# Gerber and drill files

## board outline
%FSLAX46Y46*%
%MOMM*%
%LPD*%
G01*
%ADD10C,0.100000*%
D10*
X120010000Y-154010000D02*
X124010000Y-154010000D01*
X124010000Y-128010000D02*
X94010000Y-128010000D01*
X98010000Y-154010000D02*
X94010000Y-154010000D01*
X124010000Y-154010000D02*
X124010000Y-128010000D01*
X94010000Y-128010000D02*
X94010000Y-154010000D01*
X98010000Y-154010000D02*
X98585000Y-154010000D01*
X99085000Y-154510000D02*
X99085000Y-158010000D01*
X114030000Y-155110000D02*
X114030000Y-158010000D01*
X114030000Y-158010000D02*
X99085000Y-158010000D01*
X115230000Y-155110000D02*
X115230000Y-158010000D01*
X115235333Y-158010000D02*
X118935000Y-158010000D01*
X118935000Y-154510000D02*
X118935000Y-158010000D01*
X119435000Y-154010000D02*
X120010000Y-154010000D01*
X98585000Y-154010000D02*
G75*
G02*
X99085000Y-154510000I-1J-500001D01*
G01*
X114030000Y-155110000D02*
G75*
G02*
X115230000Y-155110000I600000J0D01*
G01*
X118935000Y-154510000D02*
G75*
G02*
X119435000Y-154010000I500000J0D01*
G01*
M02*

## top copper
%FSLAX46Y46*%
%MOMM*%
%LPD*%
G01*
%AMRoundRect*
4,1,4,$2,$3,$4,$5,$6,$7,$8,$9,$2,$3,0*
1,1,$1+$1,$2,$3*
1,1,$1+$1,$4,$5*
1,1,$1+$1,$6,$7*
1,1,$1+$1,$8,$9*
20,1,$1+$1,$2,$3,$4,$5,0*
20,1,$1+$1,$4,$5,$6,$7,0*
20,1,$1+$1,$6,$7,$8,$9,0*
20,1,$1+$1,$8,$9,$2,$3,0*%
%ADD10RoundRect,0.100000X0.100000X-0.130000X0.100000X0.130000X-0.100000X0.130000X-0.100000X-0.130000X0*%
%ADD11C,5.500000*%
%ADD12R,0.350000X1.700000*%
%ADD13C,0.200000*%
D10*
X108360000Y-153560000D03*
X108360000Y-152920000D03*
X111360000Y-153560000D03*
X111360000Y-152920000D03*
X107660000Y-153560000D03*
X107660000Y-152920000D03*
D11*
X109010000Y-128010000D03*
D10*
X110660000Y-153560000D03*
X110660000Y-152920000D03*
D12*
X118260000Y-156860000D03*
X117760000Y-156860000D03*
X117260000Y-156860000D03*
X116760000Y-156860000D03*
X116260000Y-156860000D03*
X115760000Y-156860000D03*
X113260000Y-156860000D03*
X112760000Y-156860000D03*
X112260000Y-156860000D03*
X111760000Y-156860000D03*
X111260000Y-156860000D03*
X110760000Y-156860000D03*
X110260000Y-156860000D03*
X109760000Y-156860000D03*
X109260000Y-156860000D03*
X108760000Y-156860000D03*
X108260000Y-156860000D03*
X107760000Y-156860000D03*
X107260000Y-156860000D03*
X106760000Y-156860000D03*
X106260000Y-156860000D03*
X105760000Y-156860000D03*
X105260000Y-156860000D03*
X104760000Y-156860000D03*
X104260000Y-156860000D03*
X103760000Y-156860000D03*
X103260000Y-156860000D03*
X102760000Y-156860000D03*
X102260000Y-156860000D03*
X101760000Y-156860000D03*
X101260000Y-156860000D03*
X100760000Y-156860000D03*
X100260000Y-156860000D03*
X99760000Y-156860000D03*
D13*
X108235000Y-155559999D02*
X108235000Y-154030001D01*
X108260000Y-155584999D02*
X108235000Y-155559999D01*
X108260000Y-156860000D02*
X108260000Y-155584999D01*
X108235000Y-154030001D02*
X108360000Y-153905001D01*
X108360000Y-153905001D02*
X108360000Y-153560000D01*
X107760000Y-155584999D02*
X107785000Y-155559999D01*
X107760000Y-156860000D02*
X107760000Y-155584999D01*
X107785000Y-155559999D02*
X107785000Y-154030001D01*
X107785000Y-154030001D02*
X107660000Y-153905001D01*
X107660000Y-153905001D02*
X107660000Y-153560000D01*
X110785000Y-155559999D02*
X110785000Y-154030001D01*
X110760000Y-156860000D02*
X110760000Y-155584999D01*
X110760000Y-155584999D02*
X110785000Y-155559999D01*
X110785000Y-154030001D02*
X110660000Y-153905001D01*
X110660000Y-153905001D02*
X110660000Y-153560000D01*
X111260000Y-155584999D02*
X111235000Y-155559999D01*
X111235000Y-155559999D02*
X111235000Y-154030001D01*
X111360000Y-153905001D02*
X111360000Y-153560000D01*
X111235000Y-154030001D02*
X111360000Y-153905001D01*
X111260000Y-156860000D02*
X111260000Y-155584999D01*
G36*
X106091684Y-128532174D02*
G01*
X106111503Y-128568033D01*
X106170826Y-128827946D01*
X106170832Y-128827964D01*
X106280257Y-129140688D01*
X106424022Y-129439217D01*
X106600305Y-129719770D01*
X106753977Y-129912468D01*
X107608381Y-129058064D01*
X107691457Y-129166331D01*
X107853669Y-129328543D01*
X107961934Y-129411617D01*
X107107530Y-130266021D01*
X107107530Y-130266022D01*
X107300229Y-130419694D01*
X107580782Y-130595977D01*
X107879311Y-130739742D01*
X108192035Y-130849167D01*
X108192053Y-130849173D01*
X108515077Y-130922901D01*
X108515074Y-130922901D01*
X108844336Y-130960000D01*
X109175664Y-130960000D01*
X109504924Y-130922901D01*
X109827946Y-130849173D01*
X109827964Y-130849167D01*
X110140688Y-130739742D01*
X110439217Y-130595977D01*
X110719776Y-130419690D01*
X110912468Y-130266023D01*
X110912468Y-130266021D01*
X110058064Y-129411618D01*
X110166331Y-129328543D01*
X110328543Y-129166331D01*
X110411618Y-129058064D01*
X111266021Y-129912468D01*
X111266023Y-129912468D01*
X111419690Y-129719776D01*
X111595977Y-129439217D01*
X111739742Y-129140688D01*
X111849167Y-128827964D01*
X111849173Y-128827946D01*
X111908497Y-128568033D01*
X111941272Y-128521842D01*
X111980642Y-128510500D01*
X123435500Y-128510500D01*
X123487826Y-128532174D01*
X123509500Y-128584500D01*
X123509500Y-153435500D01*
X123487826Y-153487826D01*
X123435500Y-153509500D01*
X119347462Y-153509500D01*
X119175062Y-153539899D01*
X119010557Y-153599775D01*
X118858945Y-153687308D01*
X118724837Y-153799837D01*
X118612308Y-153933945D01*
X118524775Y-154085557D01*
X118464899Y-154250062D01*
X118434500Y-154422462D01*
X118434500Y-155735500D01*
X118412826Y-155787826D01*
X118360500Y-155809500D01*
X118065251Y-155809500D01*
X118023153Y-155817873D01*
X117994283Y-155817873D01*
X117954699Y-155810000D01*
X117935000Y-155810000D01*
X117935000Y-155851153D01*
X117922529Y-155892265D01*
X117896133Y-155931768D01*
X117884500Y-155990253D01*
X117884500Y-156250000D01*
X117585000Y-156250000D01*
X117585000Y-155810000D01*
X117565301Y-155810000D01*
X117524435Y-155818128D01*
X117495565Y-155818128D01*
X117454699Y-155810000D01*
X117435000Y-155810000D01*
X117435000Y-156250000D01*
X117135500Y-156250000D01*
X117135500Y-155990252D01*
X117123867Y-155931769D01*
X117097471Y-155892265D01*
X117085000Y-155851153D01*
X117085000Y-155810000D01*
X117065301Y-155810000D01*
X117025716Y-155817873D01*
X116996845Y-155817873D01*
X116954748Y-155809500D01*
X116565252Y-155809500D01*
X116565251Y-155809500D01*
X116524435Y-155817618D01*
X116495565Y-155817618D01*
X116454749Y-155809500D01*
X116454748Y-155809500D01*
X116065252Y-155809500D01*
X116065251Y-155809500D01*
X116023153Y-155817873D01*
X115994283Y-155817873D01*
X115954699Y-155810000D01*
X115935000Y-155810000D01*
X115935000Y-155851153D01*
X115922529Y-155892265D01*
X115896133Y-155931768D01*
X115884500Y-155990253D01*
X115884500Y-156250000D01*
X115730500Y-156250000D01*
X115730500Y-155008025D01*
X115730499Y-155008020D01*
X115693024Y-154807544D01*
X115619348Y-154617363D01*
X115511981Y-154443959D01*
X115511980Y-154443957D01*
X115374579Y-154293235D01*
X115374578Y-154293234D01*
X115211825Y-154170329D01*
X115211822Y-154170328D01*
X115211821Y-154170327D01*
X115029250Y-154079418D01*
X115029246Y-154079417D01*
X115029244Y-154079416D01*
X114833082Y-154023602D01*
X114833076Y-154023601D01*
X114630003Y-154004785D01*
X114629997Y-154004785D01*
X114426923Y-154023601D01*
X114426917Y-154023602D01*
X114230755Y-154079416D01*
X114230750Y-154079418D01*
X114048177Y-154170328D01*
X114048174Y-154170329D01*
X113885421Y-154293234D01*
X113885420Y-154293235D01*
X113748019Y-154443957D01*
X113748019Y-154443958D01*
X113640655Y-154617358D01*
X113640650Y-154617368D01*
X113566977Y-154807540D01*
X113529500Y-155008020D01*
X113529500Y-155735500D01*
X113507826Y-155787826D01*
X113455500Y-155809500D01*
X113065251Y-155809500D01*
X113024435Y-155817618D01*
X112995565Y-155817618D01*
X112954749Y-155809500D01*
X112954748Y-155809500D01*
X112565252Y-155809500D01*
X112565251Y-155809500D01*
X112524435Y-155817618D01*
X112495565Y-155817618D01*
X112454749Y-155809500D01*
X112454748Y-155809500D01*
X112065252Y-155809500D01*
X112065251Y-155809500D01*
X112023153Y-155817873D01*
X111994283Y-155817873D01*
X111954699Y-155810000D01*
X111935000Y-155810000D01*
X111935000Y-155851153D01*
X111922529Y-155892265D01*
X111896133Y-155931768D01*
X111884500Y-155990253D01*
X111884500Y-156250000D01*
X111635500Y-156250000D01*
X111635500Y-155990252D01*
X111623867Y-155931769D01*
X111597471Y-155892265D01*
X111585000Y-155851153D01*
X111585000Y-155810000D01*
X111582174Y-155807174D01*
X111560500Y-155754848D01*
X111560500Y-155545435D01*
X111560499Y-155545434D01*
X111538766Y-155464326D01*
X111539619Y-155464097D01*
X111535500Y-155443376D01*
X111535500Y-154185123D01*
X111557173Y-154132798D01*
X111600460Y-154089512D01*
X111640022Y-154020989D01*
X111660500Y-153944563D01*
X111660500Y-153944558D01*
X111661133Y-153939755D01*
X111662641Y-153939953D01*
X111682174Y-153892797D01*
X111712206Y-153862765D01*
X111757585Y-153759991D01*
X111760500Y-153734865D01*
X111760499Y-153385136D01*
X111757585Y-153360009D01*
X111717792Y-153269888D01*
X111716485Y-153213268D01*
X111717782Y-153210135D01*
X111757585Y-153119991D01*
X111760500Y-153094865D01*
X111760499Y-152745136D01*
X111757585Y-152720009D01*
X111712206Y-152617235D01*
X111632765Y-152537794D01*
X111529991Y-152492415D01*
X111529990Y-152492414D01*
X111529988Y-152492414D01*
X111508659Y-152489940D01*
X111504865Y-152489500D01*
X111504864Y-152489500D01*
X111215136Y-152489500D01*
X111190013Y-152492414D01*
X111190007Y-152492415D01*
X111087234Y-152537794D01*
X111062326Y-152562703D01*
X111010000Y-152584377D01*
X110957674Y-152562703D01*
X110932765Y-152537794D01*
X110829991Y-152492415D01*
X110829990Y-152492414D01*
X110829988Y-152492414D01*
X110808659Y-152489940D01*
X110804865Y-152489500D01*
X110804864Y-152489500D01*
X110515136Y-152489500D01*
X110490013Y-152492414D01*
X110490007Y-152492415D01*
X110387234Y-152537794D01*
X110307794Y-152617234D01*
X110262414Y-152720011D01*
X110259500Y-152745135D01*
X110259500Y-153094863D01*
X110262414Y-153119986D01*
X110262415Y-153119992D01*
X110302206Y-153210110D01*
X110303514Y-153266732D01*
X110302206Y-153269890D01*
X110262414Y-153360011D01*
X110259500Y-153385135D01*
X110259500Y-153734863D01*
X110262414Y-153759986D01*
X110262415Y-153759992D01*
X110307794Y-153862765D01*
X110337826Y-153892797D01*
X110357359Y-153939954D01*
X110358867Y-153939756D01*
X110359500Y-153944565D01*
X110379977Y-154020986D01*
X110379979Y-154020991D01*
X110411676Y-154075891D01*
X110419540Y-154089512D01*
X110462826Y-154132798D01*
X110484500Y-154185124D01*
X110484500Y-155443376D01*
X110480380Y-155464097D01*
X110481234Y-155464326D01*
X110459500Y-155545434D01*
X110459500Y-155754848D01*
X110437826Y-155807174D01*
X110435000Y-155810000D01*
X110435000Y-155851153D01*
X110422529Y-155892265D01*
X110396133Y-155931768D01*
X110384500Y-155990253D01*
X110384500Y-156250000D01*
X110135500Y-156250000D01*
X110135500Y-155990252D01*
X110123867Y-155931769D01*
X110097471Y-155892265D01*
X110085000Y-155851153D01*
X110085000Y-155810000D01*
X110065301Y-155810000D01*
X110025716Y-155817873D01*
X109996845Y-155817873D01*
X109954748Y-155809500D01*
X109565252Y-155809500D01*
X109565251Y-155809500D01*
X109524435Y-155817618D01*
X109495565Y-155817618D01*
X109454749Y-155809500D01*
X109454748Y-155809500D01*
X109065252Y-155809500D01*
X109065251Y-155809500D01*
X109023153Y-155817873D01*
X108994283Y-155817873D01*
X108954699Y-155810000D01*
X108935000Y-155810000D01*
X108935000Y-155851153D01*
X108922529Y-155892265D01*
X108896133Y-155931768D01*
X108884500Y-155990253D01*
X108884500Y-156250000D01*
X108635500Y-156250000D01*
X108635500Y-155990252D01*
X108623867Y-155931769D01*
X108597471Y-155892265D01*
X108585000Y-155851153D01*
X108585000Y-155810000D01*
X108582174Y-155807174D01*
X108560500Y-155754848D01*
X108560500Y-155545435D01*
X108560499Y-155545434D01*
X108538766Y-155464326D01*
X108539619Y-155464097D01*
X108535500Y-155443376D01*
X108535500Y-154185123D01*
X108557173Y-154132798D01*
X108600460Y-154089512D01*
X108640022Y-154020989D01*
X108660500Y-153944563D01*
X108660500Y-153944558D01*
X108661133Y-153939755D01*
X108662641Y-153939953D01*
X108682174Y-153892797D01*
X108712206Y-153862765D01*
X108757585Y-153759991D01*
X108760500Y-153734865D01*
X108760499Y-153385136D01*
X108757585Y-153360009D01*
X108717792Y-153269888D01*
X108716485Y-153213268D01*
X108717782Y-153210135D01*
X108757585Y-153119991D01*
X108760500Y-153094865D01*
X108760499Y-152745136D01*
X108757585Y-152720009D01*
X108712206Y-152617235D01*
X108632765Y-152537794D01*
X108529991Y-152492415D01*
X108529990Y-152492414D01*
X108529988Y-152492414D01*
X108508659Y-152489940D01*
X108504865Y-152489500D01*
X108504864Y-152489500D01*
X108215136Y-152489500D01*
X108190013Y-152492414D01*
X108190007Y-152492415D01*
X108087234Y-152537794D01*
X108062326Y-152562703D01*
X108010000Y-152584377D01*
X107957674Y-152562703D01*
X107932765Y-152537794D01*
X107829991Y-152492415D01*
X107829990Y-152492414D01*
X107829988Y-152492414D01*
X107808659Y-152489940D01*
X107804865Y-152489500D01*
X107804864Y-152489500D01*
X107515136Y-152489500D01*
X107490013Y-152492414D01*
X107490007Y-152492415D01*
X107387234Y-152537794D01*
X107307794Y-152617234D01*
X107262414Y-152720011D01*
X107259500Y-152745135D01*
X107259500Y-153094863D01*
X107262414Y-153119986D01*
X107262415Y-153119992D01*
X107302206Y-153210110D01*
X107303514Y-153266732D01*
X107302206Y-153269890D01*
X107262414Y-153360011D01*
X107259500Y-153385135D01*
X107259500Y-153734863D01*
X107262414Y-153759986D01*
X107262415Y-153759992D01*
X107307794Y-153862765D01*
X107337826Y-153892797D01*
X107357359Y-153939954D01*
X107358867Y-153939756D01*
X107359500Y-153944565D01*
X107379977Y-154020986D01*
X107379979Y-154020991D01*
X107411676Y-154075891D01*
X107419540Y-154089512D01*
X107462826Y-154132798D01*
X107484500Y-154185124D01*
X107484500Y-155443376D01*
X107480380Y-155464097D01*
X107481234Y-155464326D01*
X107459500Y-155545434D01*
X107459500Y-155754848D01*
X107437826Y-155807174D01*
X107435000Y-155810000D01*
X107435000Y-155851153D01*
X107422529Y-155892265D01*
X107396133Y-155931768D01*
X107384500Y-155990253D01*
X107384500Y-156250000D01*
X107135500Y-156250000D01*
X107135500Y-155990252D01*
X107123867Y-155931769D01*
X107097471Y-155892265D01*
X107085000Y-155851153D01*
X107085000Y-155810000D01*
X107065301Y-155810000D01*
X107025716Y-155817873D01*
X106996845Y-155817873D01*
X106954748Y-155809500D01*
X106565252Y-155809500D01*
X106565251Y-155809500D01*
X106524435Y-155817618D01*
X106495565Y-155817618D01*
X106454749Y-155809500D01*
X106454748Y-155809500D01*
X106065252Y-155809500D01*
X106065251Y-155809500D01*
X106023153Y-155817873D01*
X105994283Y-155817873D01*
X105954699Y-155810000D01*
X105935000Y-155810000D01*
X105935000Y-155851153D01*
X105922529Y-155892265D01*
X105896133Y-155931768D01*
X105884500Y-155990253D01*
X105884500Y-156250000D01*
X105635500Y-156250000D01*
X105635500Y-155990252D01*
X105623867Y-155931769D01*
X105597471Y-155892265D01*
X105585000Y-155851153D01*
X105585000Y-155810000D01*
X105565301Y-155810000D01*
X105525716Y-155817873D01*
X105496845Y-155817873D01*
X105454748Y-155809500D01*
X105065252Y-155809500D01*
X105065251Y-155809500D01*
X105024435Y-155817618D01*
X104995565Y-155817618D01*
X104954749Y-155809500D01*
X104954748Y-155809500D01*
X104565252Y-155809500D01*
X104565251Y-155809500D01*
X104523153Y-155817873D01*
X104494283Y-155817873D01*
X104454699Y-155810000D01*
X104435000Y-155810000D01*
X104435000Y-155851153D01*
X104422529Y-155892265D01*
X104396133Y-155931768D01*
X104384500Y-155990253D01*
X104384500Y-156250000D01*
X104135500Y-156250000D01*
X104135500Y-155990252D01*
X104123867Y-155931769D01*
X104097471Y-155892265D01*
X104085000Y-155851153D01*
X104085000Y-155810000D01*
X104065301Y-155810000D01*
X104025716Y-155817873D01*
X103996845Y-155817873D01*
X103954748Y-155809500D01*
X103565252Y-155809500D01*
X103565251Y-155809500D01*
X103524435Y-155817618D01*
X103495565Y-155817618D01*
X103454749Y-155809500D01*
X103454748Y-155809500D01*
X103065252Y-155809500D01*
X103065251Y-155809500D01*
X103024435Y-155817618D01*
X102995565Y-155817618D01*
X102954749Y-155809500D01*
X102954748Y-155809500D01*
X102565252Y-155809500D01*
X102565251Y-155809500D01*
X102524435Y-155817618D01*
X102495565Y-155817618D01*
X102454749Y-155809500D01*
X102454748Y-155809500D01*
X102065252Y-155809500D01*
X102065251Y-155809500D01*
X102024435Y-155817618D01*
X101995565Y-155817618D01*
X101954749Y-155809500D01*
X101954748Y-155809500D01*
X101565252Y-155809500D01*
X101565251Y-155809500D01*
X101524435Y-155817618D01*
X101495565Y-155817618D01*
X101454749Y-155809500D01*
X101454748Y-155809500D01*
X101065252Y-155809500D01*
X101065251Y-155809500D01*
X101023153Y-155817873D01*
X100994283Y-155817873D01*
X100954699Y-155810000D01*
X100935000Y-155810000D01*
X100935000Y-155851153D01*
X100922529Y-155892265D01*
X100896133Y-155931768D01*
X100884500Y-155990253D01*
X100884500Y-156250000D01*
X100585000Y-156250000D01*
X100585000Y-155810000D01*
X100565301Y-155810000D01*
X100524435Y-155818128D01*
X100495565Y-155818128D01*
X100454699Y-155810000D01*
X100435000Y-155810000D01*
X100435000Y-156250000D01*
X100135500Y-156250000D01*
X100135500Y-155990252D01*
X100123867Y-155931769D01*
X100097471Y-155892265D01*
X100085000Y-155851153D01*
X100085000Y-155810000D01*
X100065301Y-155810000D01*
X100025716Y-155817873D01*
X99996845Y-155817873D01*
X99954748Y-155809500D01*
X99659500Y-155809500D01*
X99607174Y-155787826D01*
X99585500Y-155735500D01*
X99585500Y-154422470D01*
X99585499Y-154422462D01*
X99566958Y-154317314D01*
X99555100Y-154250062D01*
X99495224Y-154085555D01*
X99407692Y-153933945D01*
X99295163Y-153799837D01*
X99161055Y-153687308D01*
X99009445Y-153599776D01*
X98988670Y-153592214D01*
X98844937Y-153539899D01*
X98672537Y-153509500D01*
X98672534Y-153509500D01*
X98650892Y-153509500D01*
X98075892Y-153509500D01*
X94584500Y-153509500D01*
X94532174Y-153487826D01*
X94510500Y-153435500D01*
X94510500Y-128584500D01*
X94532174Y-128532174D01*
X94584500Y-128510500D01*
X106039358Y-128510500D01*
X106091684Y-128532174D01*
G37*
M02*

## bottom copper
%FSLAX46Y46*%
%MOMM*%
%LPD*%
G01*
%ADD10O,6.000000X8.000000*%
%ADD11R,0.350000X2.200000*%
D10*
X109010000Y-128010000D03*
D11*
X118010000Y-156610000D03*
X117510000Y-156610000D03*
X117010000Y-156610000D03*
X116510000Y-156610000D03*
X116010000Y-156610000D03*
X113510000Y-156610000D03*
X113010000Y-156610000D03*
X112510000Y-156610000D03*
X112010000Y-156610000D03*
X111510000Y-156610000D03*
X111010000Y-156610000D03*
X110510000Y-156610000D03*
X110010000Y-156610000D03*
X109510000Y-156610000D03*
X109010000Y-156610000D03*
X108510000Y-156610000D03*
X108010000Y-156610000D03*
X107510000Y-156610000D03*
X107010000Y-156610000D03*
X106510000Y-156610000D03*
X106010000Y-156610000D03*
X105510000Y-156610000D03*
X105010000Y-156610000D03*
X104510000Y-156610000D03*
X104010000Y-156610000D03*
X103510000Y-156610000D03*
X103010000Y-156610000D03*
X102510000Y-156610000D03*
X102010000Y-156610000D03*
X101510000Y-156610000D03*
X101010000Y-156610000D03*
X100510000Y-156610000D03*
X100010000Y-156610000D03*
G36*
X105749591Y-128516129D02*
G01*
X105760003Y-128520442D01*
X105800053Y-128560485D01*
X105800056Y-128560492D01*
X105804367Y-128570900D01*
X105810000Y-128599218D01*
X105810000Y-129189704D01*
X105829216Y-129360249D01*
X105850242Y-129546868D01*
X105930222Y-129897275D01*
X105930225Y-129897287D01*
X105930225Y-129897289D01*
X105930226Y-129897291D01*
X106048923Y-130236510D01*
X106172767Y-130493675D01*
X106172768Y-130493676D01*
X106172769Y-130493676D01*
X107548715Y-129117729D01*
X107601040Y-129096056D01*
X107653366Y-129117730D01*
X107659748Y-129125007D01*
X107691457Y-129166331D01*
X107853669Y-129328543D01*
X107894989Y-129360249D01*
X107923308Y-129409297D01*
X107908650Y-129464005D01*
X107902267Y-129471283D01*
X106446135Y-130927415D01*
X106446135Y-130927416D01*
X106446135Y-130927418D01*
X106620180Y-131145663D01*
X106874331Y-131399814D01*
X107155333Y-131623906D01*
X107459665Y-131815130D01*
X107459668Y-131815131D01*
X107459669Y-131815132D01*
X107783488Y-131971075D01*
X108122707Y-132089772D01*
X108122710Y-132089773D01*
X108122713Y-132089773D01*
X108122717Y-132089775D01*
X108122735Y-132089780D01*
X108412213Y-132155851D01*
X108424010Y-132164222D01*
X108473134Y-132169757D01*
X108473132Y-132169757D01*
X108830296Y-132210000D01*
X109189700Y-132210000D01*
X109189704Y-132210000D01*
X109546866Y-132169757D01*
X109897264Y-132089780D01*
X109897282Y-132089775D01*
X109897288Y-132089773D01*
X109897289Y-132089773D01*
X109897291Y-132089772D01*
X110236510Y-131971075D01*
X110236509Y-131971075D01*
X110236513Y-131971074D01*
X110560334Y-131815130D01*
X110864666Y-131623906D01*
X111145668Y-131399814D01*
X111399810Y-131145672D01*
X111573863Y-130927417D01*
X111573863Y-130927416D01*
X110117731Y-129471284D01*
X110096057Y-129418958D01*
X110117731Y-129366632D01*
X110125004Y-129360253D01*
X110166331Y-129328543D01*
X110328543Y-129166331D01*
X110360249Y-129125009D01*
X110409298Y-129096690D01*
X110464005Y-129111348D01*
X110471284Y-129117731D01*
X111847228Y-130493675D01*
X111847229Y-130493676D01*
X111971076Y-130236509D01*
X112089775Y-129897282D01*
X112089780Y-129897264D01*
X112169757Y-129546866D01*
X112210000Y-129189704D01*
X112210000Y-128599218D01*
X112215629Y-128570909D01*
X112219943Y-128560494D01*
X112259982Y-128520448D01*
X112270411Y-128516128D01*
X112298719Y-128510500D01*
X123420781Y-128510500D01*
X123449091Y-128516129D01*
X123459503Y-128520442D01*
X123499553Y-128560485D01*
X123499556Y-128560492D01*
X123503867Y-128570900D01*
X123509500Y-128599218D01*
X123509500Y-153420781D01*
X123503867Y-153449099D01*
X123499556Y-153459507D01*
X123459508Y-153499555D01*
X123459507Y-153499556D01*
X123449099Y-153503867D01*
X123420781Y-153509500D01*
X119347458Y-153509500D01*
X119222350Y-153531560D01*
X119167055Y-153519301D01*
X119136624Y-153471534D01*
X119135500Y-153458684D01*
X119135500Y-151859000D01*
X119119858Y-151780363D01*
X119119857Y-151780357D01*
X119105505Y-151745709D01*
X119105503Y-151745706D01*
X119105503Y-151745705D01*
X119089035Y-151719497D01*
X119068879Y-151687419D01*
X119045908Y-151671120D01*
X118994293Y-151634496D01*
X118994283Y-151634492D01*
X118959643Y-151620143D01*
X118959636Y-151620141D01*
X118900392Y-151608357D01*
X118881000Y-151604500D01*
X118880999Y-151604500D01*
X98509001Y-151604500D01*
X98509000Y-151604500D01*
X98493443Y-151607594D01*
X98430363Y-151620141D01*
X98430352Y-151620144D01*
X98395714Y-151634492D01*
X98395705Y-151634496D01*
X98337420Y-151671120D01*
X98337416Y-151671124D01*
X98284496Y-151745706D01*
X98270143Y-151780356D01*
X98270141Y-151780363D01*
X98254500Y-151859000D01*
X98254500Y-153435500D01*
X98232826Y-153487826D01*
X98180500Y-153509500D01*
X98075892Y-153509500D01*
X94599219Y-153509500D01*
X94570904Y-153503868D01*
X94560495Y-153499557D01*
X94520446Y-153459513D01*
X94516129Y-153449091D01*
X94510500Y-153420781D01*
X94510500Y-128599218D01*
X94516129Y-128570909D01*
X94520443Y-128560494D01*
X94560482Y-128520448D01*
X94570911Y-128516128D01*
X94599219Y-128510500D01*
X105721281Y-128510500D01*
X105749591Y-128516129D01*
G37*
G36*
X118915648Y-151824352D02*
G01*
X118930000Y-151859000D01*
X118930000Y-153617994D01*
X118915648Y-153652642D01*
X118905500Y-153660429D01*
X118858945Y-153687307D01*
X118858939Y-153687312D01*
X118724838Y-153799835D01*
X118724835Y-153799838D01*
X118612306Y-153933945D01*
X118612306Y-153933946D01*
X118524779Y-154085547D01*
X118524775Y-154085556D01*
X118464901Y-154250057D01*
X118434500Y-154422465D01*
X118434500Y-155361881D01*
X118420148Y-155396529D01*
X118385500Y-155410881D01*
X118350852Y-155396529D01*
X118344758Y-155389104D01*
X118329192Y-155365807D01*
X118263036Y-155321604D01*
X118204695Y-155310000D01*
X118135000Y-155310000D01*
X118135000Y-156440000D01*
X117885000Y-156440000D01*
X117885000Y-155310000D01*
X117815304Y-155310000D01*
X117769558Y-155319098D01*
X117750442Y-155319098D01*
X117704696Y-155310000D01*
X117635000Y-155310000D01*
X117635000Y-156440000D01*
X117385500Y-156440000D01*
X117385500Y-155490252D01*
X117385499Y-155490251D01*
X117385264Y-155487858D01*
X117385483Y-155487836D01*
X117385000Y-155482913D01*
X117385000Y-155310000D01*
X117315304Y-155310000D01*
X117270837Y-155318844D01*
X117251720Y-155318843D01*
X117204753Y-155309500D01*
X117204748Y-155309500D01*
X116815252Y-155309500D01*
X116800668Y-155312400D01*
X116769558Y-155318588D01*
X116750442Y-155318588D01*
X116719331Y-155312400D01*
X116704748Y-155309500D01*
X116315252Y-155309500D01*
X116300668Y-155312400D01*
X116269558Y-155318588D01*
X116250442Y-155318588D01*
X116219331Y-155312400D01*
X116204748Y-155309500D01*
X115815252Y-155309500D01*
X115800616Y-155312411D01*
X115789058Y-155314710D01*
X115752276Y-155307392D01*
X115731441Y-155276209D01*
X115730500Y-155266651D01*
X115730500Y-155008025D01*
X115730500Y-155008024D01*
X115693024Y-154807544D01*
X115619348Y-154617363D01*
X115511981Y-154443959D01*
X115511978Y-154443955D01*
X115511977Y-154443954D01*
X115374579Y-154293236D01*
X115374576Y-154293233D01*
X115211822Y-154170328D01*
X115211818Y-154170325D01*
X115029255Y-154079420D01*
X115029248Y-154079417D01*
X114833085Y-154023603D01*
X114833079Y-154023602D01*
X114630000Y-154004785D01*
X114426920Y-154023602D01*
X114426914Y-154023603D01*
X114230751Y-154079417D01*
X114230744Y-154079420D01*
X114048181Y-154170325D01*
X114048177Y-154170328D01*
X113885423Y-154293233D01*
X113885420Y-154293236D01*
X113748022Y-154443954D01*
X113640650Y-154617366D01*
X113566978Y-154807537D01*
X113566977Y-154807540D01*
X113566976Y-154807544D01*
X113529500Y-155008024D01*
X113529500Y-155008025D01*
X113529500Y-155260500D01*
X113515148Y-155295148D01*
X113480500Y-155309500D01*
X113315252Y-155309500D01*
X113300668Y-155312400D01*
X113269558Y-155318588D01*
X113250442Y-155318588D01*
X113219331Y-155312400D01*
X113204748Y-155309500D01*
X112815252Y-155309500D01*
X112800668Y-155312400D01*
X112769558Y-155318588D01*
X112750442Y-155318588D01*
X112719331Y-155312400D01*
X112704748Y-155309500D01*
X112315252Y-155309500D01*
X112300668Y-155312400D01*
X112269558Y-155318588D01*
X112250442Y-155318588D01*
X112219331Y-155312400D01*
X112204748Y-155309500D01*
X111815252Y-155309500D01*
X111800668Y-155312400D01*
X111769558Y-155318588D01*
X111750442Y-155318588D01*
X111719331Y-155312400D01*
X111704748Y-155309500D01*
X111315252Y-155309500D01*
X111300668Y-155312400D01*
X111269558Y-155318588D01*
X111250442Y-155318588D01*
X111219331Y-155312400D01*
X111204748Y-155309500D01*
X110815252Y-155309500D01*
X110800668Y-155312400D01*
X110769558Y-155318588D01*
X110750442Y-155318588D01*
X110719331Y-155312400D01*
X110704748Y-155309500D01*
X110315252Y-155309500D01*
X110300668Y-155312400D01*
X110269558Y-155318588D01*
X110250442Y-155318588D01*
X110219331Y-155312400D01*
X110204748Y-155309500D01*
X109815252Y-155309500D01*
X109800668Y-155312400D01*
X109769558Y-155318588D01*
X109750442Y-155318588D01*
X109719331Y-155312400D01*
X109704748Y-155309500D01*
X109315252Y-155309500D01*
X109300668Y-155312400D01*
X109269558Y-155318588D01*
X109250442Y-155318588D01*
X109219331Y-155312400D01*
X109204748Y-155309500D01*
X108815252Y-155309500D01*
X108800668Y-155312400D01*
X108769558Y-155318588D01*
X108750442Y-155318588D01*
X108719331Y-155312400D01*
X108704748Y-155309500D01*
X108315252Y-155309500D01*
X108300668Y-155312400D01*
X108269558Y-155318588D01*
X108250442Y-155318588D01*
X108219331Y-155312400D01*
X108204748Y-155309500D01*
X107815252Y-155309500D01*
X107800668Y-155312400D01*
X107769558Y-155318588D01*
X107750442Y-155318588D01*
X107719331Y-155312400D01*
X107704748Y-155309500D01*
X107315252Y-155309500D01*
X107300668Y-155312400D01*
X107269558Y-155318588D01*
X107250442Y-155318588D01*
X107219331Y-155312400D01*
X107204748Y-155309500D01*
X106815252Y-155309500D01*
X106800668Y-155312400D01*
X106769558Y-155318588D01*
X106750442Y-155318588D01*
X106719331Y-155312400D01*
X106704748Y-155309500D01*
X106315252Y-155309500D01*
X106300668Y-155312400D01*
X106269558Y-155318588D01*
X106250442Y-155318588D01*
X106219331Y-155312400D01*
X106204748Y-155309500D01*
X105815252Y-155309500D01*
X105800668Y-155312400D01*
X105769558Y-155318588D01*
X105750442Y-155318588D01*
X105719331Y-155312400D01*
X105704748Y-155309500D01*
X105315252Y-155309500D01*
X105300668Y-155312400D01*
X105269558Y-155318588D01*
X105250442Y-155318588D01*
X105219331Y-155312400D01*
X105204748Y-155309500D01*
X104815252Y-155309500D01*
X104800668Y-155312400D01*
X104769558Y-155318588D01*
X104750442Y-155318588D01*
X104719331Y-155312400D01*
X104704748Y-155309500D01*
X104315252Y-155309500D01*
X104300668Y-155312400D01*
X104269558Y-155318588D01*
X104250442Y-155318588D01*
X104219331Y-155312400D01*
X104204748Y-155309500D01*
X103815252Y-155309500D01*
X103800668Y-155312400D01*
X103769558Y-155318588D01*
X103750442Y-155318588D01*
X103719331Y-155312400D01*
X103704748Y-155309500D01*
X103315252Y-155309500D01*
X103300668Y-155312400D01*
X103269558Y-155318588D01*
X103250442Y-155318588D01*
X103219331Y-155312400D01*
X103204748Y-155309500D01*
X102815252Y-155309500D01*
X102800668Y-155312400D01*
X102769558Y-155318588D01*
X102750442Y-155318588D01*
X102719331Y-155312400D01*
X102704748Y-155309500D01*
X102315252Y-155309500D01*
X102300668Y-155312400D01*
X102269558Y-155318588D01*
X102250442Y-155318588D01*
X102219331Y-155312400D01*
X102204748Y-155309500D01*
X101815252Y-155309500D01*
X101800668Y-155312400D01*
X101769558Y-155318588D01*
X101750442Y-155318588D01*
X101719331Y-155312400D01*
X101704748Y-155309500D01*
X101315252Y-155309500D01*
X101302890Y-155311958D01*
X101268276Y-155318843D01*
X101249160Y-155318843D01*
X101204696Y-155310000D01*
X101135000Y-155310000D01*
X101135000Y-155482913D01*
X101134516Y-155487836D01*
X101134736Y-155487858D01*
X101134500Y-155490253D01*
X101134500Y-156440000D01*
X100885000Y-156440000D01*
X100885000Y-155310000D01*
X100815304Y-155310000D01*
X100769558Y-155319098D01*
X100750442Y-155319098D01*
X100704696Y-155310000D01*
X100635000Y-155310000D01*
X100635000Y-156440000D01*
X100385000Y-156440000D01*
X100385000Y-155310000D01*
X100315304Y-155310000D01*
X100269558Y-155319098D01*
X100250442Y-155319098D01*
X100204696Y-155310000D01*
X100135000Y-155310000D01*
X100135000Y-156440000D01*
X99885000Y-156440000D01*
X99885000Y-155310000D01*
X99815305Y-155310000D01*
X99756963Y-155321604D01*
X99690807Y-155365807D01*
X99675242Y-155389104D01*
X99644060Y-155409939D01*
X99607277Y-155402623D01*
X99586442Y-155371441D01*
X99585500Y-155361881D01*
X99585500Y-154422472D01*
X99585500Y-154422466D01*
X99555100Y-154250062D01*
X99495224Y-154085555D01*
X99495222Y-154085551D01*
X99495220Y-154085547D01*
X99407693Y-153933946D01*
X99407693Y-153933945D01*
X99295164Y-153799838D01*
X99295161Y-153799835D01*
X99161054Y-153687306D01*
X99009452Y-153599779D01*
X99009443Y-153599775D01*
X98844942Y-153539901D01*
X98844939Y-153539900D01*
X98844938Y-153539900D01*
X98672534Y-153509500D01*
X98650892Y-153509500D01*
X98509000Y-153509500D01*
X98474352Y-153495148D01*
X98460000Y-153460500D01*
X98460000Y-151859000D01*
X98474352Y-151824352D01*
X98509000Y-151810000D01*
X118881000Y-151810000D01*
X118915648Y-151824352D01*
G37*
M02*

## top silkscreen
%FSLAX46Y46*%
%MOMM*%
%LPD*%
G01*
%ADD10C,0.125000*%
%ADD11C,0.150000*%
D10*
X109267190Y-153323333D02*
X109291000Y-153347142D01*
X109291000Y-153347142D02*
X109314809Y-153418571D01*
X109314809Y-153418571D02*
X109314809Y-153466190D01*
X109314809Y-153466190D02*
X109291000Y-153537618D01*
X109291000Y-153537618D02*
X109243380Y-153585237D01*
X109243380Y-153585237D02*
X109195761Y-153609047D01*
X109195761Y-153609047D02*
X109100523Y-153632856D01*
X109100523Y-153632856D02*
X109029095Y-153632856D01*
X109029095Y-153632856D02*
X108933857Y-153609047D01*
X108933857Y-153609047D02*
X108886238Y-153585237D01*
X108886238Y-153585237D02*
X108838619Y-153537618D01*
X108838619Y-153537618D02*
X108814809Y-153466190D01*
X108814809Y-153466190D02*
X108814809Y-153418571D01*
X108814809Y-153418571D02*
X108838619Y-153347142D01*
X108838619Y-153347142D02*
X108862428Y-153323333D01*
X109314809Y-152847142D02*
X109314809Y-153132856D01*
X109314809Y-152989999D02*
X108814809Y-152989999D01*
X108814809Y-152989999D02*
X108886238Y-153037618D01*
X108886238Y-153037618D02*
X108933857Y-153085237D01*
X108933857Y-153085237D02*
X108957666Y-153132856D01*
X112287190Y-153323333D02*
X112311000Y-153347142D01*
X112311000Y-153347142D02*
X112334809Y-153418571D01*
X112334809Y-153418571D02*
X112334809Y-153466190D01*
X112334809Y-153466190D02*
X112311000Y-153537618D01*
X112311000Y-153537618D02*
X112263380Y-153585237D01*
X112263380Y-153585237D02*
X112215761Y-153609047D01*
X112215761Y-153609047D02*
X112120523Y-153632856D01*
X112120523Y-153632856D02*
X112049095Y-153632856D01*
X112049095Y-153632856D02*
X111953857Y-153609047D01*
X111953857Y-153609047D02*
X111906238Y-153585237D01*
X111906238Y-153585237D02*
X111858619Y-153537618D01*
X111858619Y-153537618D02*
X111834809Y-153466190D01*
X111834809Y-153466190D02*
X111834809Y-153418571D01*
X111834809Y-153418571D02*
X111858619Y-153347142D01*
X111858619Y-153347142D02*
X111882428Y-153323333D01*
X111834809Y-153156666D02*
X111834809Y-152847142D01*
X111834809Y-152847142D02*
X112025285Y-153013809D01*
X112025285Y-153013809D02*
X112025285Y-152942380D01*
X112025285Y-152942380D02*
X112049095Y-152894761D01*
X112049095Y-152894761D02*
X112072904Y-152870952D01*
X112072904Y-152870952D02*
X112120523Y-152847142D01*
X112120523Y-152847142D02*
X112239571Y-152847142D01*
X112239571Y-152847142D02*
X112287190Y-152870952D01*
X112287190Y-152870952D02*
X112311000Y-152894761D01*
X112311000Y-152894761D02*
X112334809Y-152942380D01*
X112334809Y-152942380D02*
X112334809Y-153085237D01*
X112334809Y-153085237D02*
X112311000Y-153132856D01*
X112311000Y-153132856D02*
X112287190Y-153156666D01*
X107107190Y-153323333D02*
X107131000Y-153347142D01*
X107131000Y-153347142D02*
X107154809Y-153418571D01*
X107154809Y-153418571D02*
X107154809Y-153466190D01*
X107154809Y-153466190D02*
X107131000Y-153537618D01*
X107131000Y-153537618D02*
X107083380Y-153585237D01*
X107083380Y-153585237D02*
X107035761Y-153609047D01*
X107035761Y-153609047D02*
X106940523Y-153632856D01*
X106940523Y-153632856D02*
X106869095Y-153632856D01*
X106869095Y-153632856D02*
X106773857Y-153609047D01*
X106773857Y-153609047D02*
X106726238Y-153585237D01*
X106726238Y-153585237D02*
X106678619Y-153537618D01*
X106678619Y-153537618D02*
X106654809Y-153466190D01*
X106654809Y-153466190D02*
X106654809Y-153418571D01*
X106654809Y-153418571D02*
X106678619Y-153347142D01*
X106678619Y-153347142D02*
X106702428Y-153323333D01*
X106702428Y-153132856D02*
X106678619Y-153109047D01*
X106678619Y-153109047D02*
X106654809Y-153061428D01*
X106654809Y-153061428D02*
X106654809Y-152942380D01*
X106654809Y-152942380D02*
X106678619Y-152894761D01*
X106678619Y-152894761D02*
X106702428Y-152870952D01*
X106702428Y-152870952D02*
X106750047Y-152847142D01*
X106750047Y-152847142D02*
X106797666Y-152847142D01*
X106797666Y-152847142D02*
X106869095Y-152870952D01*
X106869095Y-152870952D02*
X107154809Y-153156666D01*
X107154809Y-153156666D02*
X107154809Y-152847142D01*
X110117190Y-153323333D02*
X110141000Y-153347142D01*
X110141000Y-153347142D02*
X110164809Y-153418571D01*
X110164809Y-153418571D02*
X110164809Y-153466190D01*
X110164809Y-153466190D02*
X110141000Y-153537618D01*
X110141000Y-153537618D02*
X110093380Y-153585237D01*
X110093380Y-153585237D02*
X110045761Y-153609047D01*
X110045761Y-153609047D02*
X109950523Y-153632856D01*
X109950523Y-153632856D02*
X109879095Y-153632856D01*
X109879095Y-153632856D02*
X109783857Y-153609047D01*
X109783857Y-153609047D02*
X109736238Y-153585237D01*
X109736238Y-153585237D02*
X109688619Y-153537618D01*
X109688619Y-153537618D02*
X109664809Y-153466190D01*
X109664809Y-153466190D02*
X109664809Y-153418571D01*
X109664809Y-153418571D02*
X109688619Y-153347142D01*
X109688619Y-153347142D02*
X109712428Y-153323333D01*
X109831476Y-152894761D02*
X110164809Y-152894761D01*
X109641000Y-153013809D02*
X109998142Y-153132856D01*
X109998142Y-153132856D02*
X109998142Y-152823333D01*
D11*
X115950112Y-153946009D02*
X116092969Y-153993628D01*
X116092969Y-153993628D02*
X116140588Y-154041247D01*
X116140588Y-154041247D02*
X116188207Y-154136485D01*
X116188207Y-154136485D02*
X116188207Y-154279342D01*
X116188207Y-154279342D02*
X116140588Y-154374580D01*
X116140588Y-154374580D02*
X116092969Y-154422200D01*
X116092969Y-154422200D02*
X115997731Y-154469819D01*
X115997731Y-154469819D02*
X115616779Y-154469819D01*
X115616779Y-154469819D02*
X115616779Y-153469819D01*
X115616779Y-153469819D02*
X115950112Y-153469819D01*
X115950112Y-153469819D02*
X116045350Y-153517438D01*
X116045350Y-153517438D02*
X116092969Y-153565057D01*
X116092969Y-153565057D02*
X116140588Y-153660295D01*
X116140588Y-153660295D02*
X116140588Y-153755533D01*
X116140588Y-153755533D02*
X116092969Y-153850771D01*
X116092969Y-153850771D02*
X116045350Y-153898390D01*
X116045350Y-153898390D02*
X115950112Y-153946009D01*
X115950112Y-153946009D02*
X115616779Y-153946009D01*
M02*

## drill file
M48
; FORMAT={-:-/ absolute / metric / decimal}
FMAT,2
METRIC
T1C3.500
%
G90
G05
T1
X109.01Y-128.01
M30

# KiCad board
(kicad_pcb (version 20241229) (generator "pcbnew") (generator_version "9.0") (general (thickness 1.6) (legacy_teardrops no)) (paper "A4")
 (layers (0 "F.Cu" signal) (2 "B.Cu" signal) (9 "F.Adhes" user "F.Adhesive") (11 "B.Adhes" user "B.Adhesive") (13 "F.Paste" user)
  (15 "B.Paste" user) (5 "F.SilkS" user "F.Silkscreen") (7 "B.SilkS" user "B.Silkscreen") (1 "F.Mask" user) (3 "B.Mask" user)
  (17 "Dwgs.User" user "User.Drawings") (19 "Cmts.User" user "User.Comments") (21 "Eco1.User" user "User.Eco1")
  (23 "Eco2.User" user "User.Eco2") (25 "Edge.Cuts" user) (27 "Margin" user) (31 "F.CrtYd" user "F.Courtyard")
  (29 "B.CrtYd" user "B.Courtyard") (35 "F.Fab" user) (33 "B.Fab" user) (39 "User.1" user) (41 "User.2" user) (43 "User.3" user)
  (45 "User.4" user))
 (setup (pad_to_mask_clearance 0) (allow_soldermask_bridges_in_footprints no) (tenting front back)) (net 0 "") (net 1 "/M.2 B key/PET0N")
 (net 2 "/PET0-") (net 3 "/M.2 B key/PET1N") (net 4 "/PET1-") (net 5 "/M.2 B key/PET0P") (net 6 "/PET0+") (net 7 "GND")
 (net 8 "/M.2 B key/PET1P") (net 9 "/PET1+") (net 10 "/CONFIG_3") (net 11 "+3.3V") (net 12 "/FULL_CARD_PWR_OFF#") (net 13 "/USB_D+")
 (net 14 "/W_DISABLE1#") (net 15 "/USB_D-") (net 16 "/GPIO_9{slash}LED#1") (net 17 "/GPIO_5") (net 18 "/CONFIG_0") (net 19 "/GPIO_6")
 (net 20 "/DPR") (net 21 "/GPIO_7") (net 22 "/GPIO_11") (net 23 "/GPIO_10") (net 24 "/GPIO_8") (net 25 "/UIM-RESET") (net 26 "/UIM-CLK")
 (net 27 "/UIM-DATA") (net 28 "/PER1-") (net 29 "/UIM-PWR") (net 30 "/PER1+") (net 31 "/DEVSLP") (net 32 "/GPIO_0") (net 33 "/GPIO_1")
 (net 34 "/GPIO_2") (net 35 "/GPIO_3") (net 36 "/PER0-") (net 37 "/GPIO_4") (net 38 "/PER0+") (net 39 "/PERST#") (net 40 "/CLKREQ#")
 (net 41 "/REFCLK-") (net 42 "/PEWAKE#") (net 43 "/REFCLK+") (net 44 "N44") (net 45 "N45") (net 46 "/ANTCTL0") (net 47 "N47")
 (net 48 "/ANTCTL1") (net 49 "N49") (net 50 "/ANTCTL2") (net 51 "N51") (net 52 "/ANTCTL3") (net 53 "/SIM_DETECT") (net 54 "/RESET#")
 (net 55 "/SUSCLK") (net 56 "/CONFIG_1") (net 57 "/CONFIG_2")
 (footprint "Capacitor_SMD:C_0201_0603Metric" (layer "F.Cu") (at 108.36 153.24 90)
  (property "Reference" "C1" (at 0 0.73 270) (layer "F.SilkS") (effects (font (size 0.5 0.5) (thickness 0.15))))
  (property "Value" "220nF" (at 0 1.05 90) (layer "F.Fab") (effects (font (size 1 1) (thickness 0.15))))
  (pad "" smd roundrect (at -0.345 0 90) (size 0.318 0.36) (layers "F.Paste") (roundrect_rratio 0.25))
  (pad "" smd roundrect (at 0.345 0 90) (size 0.318 0.36) (layers "F.Paste") (roundrect_rratio 0.25))
  (pad "1" smd roundrect (at -0.32 0 90) (size 0.46 0.4) (layers "F.Cu" "F.Mask") (roundrect_rratio 0.25) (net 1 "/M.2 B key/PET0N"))
  (pad "2" smd roundrect (at 0.32 0 90) (size 0.46 0.4) (layers "F.Cu" "F.Mask") (roundrect_rratio 0.25) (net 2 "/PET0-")))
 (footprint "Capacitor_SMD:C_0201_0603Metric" (layer "F.Cu") (at 111.36 153.24 90)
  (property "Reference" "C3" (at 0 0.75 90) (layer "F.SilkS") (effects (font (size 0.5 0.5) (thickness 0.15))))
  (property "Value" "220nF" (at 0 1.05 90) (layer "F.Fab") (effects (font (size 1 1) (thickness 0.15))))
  (pad "" smd roundrect (at -0.345 0 90) (size 0.318 0.36) (layers "F.Paste") (roundrect_rratio 0.25))
  (pad "" smd roundrect (at 0.345 0 90) (size 0.318 0.36) (layers "F.Paste") (roundrect_rratio 0.25))
  (pad "1" smd roundrect (at -0.32 0 90) (size 0.46 0.4) (layers "F.Cu" "F.Mask") (roundrect_rratio 0.25) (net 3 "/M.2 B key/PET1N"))
  (pad "2" smd roundrect (at 0.32 0 90) (size 0.46 0.4) (layers "F.Cu" "F.Mask") (roundrect_rratio 0.25) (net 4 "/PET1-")))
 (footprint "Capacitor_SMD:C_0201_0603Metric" (layer "F.Cu") (at 107.66 153.24 90)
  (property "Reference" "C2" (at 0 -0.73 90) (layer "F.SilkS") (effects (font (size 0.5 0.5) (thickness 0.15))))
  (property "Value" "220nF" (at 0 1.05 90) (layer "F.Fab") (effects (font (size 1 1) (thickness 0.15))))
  (pad "" smd roundrect (at -0.345 0 90) (size 0.318 0.36) (layers "F.Paste") (roundrect_rratio 0.25))
  (pad "" smd roundrect (at 0.345 0 90) (size 0.318 0.36) (layers "F.Paste") (roundrect_rratio 0.25))
  (pad "1" smd roundrect (at -0.32 0 90) (size 0.46 0.4) (layers "F.Cu" "F.Mask") (roundrect_rratio 0.25) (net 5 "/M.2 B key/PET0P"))
  (pad "2" smd roundrect (at 0.32 0 90) (size 0.46 0.4) (layers "F.Cu" "F.Mask") (roundrect_rratio 0.25) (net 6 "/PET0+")))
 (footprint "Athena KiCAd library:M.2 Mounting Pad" (layer "F.Cu") (at 109.01 128.01)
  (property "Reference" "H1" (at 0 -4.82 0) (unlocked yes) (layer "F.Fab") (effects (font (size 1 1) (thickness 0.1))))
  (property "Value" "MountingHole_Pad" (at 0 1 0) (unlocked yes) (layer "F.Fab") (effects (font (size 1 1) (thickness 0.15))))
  (pad "1" thru_hole circle (at 0 0) (size 5.5 5.5) (drill 3.5) (layers "*.Cu" "*.Mask") (remove_unused_layers no) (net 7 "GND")
   (padstack (mode front_inner_back)
    (layer "Inner" (shape circle) (size 5.5 5.5) (zone_connect -1))
    (layer "B.Cu" (shape oval) (size 6 8) (thermal_bridge_angle 45) (zone_connect -1)))))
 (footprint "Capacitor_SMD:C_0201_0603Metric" (layer "F.Cu") (at 110.66 153.24 90)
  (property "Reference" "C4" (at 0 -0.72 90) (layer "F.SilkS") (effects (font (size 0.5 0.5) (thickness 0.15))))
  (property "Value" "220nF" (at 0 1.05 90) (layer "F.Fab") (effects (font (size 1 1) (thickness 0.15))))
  (pad "" smd roundrect (at -0.345 0 90) (size 0.318 0.36) (layers "F.Paste") (roundrect_rratio 0.25))
  (pad "" smd roundrect (at 0.345 0 90) (size 0.318 0.36) (layers "F.Paste") (roundrect_rratio 0.25))
  (pad "1" smd roundrect (at -0.32 0 90) (size 0.46 0.4) (layers "F.Cu" "F.Mask") (roundrect_rratio 0.25) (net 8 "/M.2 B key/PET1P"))
  (pad "2" smd roundrect (at 0.32 0 90) (size 0.46 0.4) (layers "F.Cu" "F.Mask") (roundrect_rratio 0.25) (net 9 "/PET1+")))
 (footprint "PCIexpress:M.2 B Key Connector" (layer "F.Cu") (at 109.01 156.9)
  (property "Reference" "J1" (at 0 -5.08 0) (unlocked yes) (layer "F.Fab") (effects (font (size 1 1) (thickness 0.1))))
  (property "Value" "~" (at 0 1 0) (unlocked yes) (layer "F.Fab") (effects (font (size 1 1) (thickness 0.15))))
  (fp_line (start -11 -2.89) (end -10.425 -2.89) (stroke (width 0.1) (type default)) (layer "Edge.Cuts"))
  (fp_line (start -9.925 -2.39) (end -9.925 1.11) (stroke (width 0.1) (type default)) (layer "Edge.Cuts"))
  (fp_line (start 5.02 -1.79) (end 5.02 1.11) (stroke (width 0.1) (type default)) (layer "Edge.Cuts"))
  (fp_line (start 5.02 1.11) (end -9.925 1.11) (stroke (width 0.1) (type default)) (layer "Edge.Cuts"))
  (fp_line (start 6.22 -1.79) (end 6.22 1.11) (stroke (width 0.1) (type default)) (layer "Edge.Cuts"))
  (fp_line (start 6.225333 1.11) (end 9.925 1.11) (stroke (width 0.1) (type default)) (layer "Edge.Cuts"))
  (fp_line (start 9.925 -2.39) (end 9.925 1.11) (stroke (width 0.1) (type default)) (layer "Edge.Cuts"))
  (fp_line (start 10.425 -2.89) (end 11 -2.89) (stroke (width 0.1) (type default)) (layer "Edge.Cuts"))
  (fp_arc (start -10.425 -2.89) (mid -10.071447 -2.743553) (end -9.925 -2.39) (stroke (width 0.1) (type default)) (layer "Edge.Cuts"))
  (fp_arc (start 5.02 -1.79) (mid 5.62 -2.39) (end 6.22 -1.79) (stroke (width 0.1) (type default)) (layer "Edge.Cuts"))
  (fp_arc (start 9.925 -2.39) (mid 10.071447 -2.743553) (end 10.425 -2.89) (stroke (width 0.1) (type default)) (layer "Edge.Cuts"))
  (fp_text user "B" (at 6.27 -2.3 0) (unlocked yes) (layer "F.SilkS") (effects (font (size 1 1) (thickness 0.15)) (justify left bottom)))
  (pad "1" smd rect (at 9.25 -0.04 180) (size 0.35 1.7) (layers "F.Cu") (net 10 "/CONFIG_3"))
  (pad "2" smd rect (at 9 -0.29 180) (size 0.35 2.2) (layers "B.Cu") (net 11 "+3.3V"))
  (pad "3" smd rect (at 8.75 -0.04 180) (size 0.35 1.7) (layers "F.Cu") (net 7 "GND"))
  (pad "4" smd rect (at 8.5 -0.29 180) (size 0.35 2.2) (layers "B.Cu") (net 11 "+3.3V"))
  (pad "5" smd rect (at 8.25 -0.04 180) (size 0.35 1.7) (layers "F.Cu") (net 7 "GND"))
  (pad "6" smd rect (at 8 -0.29 180) (size 0.35 2.2) (layers "B.Cu") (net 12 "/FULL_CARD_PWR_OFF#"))
  (pad "7" smd rect (at 7.75 -0.04 180) (size 0.35 1.7) (layers "F.Cu") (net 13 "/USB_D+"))
  (pad "8" smd rect (at 7.5 -0.29 180) (size 0.35 2.2) (layers "B.Cu") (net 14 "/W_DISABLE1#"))
  (pad "9" smd rect (at 7.25 -0.04 180) (size 0.35 1.7) (layers "F.Cu") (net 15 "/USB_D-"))
  (pad "10" smd rect (at 7 -0.29 180) (size 0.35 2.2) (layers "B.Cu") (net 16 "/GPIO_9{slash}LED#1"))
  (pad "11" smd rect (at 6.75 -0.04 180) (size 0.35 1.7) (layers "F.Cu") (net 7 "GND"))
  (pad "20" smd rect (at 4.5 -0.29 180) (size 0.35 2.2) (layers "B.Cu") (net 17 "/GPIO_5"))
  (pad "21" smd rect (at 4.25 -0.04 180) (size 0.35 1.7) (layers "F.Cu") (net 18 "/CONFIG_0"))
  (pad "22" smd rect (at 4 -0.29 180) (size 0.35 2.2) (layers "B.Cu") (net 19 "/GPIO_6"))
  (pad "23" smd rect (at 3.75 -0.04 180) (size 0.35 1.7) (layers "F.Cu") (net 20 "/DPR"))
  (pad "24" smd rect (at 3.5 -0.29 180) (size 0.35 2.2) (layers "B.Cu") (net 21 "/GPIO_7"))
  (pad "25" smd rect (at 3.25 -0.04 180) (size 0.35 1.7) (layers "F.Cu") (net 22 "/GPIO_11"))
  (pad "26" smd rect (at 3 -0.29 180) (size 0.35 2.2) (layers "B.Cu") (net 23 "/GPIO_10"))
  (pad "27" smd rect (at 2.75 -0.04 180) (size 0.35 1.7) (layers "F.Cu") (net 7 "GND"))
  (pad "28" smd rect (at 2.5 -0.29 180) (size 0.35 2.2) (layers "B.Cu") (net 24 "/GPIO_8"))
  (pad "29" smd rect (at 2.25 -0.04 180) (size 0.35 1.7) (layers "F.Cu") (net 3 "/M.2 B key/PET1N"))
  (pad "30" smd rect (at 2 -0.29 180) (size 0.35 2.2) (layers "B.Cu") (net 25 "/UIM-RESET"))
  (pad "31" smd rect (at 1.75 -0.04 180) (size 0.35 1.7) (layers "F.Cu") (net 8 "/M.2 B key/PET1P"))
  (pad "32" smd rect (at 1.5 -0.29 180) (size 0.35 2.2) (layers "B.Cu") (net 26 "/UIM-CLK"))
  (pad "33" smd rect (at 1.25 -0.04 180) (size 0.35 1.7) (layers "F.Cu") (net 7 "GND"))
  (pad "34" smd rect (at 1 -0.29 180) (size 0.35 2.2) (layers "B.Cu") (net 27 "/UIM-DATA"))
  (pad "35" smd rect (at 0.75 -0.04 180) (size 0.35 1.7) (layers "F.Cu") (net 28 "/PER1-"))
  (pad "36" smd rect (at 0.5 -0.29 180) (size 0.35 2.2) (layers "B.Cu") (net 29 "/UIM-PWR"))
  (pad "37" smd rect (at 0.25 -0.04 180) (size 0.35 1.7) (layers "F.Cu") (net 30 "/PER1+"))
  (pad "38" smd rect (at 0 -0.29 180) (size 0.35 2.2) (layers "B.Cu") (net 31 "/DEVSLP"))
  (pad "39" smd rect (at -0.25 -0.04 180) (size 0.35 1.7) (layers "F.Cu") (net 7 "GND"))
  (pad "40" smd rect (at -0.5 -0.29 180) (size 0.35 2.2) (layers "B.Cu") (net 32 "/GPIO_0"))
  (pad "41" smd rect (at -0.75 -0.04 180) (size 0.35 1.7) (layers "F.Cu") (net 1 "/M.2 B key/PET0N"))
  (pad "42" smd rect (at -1 -0.29 180) (size 0.35 2.2) (layers "B.Cu") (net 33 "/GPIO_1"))
  (pad "43" smd rect (at -1.25 -0.04 180) (size 0.35 1.7) (layers "F.Cu") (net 5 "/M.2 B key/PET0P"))
  (pad "44" smd rect (at -1.5 -0.29 180) (size 0.35 2.2) (layers "B.Cu") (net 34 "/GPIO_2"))
  (pad "45" smd rect (at -1.75 -0.04 180) (size 0.35 1.7) (layers "F.Cu") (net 7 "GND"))
  (pad "46" smd rect (at -2 -0.29 180) (size 0.35 2.2) (layers "B.Cu") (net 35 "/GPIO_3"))
  (pad "47" smd rect (at -2.25 -0.04 180) (size 0.35 1.7) (layers "F.Cu") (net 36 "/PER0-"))
  (pad "48" smd rect (at -2.5 -0.29 180) (size 0.35 2.2) (layers "B.Cu") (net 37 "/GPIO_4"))
  (pad "49" smd rect (at -2.75 -0.04 180) (size 0.35 1.7) (layers "F.Cu") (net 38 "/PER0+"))
  (pad "50" smd rect (at -3 -0.29 180) (size 0.35 2.2) (layers "B.Cu") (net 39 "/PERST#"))
  (pad "51" smd rect (at -3.25 -0.04 180) (size 0.35 1.7) (layers "F.Cu") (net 7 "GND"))
  (pad "52" smd rect (at -3.5 -0.29 180) (size 0.35 2.2) (layers "B.Cu") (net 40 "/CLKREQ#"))
  (pad "53" smd rect (at -3.75 -0.04 180) (size 0.35 1.7) (layers "F.Cu") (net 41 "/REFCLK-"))
  (pad "54" smd rect (at -4 -0.29 180) (size 0.35 2.2) (layers "B.Cu") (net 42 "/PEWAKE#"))
  (pad "55" smd rect (at -4.25 -0.04 180) (size 0.35 1.7) (layers "F.Cu") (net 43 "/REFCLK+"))
  (pad "56" smd rect (at -4.5 -0.29 180) (size 0.35 2.2) (layers "B.Cu") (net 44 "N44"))
  (pad "57" smd rect (at -4.75 -0.04 180) (size 0.35 1.7) (layers "F.Cu") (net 7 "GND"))
  (pad "58" smd rect (at -5 -0.29 180) (size 0.35 2.2) (layers "B.Cu") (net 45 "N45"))
  (pad "59" smd rect (at -5.25 -0.04 180) (size 0.35 1.7) (layers "F.Cu") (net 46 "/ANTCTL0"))
  (pad "60" smd rect (at -5.5 -0.29 180) (size 0.35 2.2) (layers "B.Cu") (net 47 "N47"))
  (pad "61" smd rect (at -5.75 -0.04 180) (size 0.35 1.7) (layers "F.Cu") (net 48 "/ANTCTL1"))
  (pad "62" smd rect (at -6 -0.29 180) (size 0.35 2.2) (layers "B.Cu") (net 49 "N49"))
  (pad "63" smd rect (at -6.25 -0.04 180) (size 0.35 1.7) (layers "F.Cu") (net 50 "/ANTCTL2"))
  (pad "64" smd rect (at -6.5 -0.29 180) (size 0.35 2.2) (layers "B.Cu") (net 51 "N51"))
  (pad "65" smd rect (at -6.75 -0.04 180) (size 0.35 1.7) (layers "F.Cu") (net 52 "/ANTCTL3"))
  (pad "66" smd rect (at -7 -0.29 180) (size 0.35 2.2) (layers "B.Cu") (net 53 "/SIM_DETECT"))
  (pad "67" smd rect (at -7.25 -0.04 180) (size 0.35 1.7) (layers "F.Cu") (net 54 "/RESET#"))
  (pad "68" smd rect (at -7.5 -0.29 180) (size 0.35 2.2) (layers "B.Cu") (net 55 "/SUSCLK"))
  (pad "69" smd rect (at -7.75 -0.04 180) (size 0.35 1.7) (layers "F.Cu") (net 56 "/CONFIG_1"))
  (pad "70" smd rect (at -8 -0.29 180) (size 0.35 2.2) (layers "B.Cu") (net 11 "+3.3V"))
  (pad "71" smd rect (at -8.25 -0.04 180) (size 0.35 1.7) (layers "F.Cu") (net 7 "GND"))
  (pad "72" smd rect (at -8.5 -0.29 180) (size 0.35 2.2) (layers "B.Cu") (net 11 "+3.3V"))
  (pad "73" smd rect (at -8.75 -0.04 180) (size 0.35 1.7) (layers "F.Cu") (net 7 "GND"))
  (pad "74" smd rect (at -9 -0.29 180) (size 0.35 2.2) (layers "B.Cu") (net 11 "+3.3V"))
  (pad "75" smd rect (at -9.25 -0.04 180) (size 0.35 1.7) (layers "F.Cu") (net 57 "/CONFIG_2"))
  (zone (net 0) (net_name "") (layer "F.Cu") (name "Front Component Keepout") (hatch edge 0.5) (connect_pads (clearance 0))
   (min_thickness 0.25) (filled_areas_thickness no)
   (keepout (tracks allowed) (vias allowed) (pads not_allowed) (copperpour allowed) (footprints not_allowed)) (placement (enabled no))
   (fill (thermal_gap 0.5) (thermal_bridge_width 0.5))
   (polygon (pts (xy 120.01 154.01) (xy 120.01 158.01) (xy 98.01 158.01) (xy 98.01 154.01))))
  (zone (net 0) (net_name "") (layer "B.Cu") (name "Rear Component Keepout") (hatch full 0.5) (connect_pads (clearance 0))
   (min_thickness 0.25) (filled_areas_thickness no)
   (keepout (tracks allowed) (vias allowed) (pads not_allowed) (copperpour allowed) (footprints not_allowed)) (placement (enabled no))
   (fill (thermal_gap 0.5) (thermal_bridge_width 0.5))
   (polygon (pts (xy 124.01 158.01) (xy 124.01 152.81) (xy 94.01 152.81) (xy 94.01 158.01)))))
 (gr_line (start 120.01 154.01) (end 124.01 154.01) (stroke (width 0.1) (type default)) (layer "Edge.Cuts"))
 (gr_line (start 124.01 128.01) (end 94.01 128.01) (stroke (width 0.1) (type default)) (layer "Edge.Cuts"))
 (gr_line (start 98.01 154.01) (end 94.01 154.01) (stroke (width 0.1) (type default)) (layer "Edge.Cuts"))
 (gr_line (start 124.01 154.01) (end 124.01 128.01) (stroke (width 0.1) (type default)) (layer "Edge.Cuts"))
 (gr_line (start 94.01 128.01) (end 94.01 154.01) (stroke (width 0.1) (type default)) (layer "Edge.Cuts"))
 (segment (start 108.235 155.559999) (end 108.235 154.030001) (width 0.2) (layer "F.Cu") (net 1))
 (segment (start 108.26 155.584999) (end 108.235 155.559999) (width 0.2) (layer "F.Cu") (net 1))
 (segment (start 108.26 156.86) (end 108.26 155.584999) (width 0.2) (layer "F.Cu") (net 1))
 (segment (start 108.235 154.030001) (end 108.36 153.905001) (width 0.2) (layer "F.Cu") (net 1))
 (segment (start 108.36 153.905001) (end 108.36 153.56) (width 0.2) (layer "F.Cu") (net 1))
 (segment (start 107.76 155.584999) (end 107.785 155.559999) (width 0.2) (layer "F.Cu") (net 5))
 (segment (start 107.76 156.86) (end 107.76 155.584999) (width 0.2) (layer "F.Cu") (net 5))
 (segment (start 107.785 155.559999) (end 107.785 154.030001) (width 0.2) (layer "F.Cu") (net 5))
 (segment (start 107.785 154.030001) (end 107.66 153.905001) (width 0.2) (layer "F.Cu") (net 5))
 (segment (start 107.66 153.905001) (end 107.66 153.56) (width 0.2) (layer "F.Cu") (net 5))
 (segment (start 110.785 155.559999) (end 110.785 154.030001) (width 0.2) (layer "F.Cu") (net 8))
 (segment (start 110.76 156.86) (end 110.76 155.584999) (width 0.2) (layer "F.Cu") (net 8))
 (segment (start 110.76 155.584999) (end 110.785 155.559999) (width 0.2) (layer "F.Cu") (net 8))
 (segment (start 110.785 154.030001) (end 110.66 153.905001) (width 0.2) (layer "F.Cu") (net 8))
 (segment (start 110.66 153.905001) (end 110.66 153.56) (width 0.2) (layer "F.Cu") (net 8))
 (segment (start 111.26 155.584999) (end 111.235 155.559999) (width 0.2) (layer "F.Cu") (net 3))
 (segment (start 111.235 155.559999) (end 111.235 154.030001) (width 0.2) (layer "F.Cu") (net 3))
 (segment (start 111.36 153.905001) (end 111.36 153.56) (width 0.2) (layer "F.Cu") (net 3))
 (segment (start 111.235 154.030001) (end 111.36 153.905001) (width 0.2) (layer "F.Cu") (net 3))
 (segment (start 111.26 156.86) (end 111.26 155.584999) (width 0.2) (layer "F.Cu") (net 3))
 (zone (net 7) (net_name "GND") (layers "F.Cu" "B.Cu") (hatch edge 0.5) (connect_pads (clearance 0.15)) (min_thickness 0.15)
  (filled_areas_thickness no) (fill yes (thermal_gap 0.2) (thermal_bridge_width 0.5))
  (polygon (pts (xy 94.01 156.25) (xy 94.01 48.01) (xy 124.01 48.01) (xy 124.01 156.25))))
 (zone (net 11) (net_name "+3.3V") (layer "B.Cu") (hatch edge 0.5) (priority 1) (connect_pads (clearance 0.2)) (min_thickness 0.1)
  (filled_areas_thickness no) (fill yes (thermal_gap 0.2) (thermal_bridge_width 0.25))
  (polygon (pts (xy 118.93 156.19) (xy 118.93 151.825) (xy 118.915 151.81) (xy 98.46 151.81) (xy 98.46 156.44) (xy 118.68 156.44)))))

